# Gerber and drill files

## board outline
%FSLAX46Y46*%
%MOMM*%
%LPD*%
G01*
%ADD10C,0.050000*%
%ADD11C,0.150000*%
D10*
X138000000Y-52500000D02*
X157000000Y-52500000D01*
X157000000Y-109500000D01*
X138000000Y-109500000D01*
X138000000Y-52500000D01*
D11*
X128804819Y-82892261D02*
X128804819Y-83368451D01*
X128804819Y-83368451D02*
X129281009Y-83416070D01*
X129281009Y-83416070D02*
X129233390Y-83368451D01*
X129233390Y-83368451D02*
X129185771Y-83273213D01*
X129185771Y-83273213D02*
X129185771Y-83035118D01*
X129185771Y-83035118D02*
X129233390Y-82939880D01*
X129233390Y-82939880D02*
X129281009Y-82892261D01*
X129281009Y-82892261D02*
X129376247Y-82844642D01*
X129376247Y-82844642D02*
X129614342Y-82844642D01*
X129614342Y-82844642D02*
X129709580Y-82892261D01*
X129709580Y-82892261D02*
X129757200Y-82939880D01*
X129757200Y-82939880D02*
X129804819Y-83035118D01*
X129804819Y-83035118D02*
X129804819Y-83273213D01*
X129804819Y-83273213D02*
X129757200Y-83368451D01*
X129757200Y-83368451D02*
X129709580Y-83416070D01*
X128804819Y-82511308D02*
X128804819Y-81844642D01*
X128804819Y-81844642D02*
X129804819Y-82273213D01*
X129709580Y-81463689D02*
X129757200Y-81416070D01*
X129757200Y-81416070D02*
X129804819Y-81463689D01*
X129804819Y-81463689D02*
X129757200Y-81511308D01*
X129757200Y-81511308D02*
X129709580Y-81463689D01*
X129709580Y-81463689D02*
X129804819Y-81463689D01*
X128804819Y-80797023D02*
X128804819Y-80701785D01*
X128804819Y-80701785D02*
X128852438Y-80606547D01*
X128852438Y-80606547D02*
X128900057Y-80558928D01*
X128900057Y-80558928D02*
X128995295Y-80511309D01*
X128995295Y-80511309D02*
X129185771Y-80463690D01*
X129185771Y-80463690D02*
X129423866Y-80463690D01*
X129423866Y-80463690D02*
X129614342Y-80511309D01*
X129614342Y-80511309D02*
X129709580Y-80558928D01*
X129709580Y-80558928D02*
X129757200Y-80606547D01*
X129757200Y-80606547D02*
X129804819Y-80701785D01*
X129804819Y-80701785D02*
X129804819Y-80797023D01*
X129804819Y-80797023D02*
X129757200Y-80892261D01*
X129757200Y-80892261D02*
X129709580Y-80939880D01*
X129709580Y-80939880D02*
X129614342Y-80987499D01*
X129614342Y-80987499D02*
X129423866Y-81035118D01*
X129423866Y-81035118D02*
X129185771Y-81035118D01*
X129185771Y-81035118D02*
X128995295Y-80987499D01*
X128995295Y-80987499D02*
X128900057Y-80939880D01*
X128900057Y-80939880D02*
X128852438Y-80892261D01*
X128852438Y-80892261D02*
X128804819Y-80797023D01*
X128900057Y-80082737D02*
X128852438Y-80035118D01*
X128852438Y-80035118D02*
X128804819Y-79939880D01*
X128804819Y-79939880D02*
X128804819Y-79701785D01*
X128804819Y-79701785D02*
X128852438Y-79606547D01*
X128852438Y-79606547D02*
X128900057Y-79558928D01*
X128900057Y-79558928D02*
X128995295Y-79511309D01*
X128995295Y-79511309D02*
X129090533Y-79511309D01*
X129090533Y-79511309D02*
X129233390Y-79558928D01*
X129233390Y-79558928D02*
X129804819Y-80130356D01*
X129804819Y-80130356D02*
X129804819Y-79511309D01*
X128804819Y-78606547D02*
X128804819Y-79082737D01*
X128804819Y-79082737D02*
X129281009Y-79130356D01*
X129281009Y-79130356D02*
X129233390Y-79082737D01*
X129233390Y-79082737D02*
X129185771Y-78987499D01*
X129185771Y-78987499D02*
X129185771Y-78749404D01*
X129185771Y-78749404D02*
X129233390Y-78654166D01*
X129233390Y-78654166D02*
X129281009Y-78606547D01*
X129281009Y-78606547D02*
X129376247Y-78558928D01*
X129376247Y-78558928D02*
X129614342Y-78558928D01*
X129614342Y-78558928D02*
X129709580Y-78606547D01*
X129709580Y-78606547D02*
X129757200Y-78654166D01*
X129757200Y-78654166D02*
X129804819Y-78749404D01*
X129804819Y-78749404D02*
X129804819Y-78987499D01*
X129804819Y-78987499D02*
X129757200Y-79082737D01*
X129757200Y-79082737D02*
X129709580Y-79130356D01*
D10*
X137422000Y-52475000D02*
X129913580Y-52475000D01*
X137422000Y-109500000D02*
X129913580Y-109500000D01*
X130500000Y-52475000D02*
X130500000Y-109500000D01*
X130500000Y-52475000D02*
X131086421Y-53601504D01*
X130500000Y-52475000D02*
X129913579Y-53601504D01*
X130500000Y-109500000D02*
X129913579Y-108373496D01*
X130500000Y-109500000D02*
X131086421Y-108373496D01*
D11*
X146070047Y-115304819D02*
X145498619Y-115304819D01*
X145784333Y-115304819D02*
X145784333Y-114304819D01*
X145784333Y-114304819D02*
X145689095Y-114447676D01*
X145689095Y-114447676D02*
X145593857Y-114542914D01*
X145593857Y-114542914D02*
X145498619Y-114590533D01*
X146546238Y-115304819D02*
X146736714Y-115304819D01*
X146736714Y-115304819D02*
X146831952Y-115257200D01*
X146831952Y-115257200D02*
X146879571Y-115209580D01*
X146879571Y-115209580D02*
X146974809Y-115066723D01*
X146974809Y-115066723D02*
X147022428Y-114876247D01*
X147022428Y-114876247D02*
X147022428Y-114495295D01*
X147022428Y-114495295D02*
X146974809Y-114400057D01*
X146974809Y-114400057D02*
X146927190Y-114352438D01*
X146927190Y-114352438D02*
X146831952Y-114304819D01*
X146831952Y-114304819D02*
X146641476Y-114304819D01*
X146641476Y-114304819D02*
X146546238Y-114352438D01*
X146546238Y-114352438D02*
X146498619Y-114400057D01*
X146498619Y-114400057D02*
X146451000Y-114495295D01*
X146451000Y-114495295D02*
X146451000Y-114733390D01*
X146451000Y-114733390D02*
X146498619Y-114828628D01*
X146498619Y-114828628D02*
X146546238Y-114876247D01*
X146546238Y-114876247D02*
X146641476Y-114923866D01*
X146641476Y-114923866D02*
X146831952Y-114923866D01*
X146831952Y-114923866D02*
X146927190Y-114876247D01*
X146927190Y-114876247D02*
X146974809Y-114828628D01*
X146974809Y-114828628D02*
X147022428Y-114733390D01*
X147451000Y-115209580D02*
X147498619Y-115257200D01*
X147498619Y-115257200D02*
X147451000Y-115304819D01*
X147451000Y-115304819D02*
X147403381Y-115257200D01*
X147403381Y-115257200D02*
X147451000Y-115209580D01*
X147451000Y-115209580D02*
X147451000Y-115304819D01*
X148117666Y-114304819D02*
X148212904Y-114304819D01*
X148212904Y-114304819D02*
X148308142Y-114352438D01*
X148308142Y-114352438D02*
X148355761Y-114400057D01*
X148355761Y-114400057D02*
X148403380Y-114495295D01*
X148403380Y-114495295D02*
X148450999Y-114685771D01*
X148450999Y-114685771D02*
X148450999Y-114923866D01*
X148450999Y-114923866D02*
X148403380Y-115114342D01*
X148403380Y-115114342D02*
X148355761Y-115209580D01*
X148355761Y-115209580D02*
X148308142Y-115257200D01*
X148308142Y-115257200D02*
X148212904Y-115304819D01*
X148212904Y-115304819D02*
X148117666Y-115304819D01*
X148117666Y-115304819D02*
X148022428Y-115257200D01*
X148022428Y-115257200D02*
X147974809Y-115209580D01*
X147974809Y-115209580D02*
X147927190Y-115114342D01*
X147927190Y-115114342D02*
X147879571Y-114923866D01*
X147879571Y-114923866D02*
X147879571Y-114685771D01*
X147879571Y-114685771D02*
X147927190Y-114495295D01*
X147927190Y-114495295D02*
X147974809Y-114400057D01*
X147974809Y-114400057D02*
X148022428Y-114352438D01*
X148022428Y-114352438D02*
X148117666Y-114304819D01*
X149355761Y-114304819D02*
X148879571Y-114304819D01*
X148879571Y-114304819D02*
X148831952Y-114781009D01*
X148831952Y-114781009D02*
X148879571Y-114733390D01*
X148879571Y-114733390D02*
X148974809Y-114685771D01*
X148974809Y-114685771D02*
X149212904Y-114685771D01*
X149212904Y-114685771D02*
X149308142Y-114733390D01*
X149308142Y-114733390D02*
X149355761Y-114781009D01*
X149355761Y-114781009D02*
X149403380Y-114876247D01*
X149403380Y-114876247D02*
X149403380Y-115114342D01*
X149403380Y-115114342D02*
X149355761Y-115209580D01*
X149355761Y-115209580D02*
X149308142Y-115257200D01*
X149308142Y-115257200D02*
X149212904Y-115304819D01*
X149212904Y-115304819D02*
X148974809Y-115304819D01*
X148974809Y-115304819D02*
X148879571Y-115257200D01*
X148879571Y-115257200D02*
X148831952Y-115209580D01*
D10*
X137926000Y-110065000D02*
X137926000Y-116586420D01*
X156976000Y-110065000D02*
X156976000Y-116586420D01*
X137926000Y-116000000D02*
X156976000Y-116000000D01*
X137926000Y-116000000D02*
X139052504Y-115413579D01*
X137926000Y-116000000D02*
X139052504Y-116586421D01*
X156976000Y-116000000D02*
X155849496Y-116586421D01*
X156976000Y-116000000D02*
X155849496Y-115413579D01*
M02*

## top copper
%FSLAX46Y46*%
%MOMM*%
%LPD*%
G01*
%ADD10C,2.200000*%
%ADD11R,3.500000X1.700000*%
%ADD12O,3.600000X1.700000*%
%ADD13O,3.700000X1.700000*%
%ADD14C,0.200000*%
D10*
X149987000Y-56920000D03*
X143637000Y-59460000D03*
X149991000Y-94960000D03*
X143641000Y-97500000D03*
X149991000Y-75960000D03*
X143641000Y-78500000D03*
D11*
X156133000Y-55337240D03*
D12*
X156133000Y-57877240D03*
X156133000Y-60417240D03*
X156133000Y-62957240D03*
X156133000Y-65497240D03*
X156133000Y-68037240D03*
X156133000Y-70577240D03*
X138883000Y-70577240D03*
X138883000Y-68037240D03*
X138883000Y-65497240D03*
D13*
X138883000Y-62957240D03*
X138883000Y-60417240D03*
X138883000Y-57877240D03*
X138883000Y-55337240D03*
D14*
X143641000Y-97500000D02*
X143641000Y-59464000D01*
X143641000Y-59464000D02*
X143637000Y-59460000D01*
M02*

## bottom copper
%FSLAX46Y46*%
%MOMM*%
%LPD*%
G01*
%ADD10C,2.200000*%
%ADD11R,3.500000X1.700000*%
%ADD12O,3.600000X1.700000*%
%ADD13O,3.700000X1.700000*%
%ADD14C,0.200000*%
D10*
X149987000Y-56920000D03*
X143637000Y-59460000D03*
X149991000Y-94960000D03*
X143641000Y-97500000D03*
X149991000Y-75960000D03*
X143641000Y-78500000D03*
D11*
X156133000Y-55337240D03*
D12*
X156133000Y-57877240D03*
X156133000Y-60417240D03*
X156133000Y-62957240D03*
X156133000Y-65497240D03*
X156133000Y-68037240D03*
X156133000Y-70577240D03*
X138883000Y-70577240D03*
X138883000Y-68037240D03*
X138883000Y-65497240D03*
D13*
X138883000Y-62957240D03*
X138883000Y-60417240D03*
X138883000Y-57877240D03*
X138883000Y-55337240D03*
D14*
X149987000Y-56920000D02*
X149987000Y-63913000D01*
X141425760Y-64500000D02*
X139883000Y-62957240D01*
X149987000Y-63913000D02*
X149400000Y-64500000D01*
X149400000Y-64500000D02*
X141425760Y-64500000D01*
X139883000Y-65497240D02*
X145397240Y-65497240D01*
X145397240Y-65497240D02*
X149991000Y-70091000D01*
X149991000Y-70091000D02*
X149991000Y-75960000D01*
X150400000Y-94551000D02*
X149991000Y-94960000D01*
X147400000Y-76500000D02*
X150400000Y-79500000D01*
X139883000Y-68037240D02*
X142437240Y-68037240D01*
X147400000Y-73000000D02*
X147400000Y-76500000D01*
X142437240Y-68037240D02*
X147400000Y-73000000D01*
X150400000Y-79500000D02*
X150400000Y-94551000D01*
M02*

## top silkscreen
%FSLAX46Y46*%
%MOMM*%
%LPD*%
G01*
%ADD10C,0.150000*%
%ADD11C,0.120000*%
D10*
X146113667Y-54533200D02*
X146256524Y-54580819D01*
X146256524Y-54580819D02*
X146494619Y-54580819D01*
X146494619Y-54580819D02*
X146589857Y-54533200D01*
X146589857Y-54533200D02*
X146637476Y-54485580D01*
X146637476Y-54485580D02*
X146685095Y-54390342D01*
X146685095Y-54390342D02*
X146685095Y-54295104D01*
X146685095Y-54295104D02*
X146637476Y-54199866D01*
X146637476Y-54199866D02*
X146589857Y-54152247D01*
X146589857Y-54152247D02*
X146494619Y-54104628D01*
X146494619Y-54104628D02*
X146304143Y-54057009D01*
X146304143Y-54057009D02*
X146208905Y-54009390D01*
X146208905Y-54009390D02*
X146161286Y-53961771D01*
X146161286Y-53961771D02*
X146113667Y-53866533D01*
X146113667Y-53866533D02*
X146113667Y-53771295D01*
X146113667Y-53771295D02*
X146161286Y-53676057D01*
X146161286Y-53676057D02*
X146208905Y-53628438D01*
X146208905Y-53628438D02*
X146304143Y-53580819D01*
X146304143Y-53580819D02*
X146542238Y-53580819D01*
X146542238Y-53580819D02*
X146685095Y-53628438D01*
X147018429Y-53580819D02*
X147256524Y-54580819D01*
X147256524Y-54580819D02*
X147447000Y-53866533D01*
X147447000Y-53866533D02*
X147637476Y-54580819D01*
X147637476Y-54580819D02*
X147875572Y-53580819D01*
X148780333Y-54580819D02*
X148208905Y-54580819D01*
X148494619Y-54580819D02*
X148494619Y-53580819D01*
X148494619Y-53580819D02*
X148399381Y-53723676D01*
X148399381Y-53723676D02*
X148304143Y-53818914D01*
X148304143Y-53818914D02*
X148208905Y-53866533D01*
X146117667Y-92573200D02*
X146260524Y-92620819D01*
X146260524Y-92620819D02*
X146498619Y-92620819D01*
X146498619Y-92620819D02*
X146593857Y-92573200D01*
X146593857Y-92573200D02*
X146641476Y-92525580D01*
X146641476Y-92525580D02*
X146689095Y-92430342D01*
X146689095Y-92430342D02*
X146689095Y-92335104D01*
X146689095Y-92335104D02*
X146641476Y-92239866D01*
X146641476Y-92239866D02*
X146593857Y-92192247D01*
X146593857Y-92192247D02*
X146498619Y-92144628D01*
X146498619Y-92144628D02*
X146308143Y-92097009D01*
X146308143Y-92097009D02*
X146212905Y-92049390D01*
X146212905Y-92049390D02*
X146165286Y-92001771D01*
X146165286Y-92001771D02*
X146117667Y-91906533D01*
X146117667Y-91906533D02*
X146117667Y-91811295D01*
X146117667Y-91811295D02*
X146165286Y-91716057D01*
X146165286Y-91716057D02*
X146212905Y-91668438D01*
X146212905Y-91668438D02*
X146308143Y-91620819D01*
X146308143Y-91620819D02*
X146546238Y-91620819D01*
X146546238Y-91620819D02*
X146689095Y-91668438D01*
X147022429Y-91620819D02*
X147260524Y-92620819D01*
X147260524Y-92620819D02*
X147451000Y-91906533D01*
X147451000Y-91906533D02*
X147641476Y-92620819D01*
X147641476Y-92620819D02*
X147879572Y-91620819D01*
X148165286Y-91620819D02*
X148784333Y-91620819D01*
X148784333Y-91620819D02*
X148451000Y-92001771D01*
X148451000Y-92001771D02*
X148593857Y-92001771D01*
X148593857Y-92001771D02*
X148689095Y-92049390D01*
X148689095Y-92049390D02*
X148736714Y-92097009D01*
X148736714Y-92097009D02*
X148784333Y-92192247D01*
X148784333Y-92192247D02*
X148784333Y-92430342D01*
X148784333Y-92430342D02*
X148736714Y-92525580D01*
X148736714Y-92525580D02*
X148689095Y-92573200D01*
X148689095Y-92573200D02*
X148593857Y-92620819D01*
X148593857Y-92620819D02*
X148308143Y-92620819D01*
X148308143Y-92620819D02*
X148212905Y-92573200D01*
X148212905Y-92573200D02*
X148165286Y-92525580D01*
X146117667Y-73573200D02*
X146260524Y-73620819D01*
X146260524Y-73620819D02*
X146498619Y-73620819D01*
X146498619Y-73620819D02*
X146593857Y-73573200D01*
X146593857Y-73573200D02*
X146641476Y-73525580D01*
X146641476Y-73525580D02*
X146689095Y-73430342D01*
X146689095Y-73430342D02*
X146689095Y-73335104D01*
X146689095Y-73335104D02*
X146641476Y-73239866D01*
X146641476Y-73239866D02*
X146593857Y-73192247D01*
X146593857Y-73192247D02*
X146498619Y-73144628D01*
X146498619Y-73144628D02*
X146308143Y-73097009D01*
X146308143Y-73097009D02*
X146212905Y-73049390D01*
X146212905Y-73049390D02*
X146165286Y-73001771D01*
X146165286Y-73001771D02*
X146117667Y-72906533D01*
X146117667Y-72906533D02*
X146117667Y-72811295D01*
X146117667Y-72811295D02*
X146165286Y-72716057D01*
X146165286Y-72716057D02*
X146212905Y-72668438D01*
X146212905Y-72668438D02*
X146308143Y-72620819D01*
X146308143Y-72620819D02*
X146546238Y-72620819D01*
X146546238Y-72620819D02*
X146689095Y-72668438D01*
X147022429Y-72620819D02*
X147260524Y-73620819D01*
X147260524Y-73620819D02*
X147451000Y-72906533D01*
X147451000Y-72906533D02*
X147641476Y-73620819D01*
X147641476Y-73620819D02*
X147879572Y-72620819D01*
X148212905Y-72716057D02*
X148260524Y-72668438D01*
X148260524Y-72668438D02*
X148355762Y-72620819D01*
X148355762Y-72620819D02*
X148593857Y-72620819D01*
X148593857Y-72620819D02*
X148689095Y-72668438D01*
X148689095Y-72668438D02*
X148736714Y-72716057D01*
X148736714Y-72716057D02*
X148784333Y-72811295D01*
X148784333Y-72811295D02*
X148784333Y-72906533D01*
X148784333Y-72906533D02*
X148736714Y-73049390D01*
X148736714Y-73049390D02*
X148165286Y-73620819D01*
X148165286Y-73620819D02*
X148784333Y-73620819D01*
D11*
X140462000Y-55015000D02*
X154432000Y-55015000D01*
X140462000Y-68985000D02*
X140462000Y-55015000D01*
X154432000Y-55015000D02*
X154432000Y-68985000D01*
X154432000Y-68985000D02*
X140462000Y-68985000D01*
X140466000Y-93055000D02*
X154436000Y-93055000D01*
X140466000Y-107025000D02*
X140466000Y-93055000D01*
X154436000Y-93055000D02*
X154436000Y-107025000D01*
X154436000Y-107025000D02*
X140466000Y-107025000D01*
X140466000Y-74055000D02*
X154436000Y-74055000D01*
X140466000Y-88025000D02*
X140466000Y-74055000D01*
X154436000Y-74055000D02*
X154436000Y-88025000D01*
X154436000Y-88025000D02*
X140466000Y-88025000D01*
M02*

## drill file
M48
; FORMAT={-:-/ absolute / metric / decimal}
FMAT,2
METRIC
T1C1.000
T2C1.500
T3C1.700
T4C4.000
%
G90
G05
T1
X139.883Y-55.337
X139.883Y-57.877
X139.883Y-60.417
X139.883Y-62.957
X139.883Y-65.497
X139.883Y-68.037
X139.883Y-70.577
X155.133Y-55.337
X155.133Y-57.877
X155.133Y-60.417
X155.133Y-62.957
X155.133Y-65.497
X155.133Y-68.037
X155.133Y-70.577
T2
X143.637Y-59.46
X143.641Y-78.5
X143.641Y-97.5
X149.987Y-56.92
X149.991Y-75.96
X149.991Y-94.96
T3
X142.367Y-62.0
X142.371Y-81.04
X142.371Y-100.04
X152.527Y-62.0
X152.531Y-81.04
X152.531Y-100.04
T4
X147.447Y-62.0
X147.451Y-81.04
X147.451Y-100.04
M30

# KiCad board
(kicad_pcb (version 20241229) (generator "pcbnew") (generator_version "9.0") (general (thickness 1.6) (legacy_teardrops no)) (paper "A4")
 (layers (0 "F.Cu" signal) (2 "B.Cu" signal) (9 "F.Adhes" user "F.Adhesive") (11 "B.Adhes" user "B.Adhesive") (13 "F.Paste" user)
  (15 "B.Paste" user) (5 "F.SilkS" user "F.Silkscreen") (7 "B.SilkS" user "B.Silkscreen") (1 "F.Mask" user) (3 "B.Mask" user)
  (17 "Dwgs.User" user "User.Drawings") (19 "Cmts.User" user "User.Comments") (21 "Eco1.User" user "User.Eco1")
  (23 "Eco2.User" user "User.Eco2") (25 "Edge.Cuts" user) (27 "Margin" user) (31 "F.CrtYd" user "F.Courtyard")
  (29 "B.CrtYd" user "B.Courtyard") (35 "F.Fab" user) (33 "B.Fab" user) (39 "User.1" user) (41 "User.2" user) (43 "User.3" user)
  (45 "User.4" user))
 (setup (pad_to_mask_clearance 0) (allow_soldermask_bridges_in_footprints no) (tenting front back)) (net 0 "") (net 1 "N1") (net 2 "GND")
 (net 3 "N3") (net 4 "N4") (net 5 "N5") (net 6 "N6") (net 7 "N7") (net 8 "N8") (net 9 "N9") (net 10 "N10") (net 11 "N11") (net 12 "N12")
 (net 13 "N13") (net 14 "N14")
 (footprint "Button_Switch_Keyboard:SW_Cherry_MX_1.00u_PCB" (layer "F.Cu") (at 149.987 56.92)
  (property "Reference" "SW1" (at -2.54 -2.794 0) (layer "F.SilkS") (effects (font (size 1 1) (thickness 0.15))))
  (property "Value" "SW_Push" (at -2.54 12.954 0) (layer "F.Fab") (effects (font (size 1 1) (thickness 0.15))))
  (fp_line (start -9.525 -1.905) (end 4.445 -1.905) (stroke (width 0.12) (type solid)) (layer "F.SilkS"))
  (fp_line (start -9.525 12.065) (end -9.525 -1.905) (stroke (width 0.12) (type solid)) (layer "F.SilkS"))
  (fp_line (start 4.445 -1.905) (end 4.445 12.065) (stroke (width 0.12) (type solid)) (layer "F.SilkS"))
  (fp_line (start 4.445 12.065) (end -9.525 12.065) (stroke (width 0.12) (type solid)) (layer "F.SilkS"))
  (pad "" np_thru_hole circle (at -7.62 5.08) (size 1.7 1.7) (drill 1.7) (layers "*.Cu" "*.Mask"))
  (pad "" np_thru_hole circle (at -2.54 5.08) (size 4 4) (drill 4) (layers "*.Cu" "*.Mask"))
  (pad "" np_thru_hole circle (at 2.54 5.08) (size 1.7 1.7) (drill 1.7) (layers "*.Cu" "*.Mask"))
  (pad "1" thru_hole circle (at 0 0) (size 2.2 2.2) (drill 1.5) (layers "*.Cu" "*.Mask") (remove_unused_layers no) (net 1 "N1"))
  (pad "2" thru_hole circle (at -6.35 2.54) (size 2.2 2.2) (drill 1.5) (layers "*.Cu" "*.Mask") (remove_unused_layers no) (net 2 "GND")))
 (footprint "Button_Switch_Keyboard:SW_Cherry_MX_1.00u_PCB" (layer "F.Cu") (at 149.991 94.96)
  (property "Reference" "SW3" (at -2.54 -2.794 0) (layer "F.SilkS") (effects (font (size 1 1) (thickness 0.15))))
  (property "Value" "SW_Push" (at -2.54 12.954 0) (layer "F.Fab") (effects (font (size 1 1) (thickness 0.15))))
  (fp_line (start -9.525 -1.905) (end 4.445 -1.905) (stroke (width 0.12) (type solid)) (layer "F.SilkS"))
  (fp_line (start -9.525 12.065) (end -9.525 -1.905) (stroke (width 0.12) (type solid)) (layer "F.SilkS"))
  (fp_line (start 4.445 -1.905) (end 4.445 12.065) (stroke (width 0.12) (type solid)) (layer "F.SilkS"))
  (fp_line (start 4.445 12.065) (end -9.525 12.065) (stroke (width 0.12) (type solid)) (layer "F.SilkS"))
  (pad "" np_thru_hole circle (at -7.62 5.08) (size 1.7 1.7) (drill 1.7) (layers "*.Cu" "*.Mask"))
  (pad "" np_thru_hole circle (at -2.54 5.08) (size 4 4) (drill 4) (layers "*.Cu" "*.Mask"))
  (pad "" np_thru_hole circle (at 2.54 5.08) (size 1.7 1.7) (drill 1.7) (layers "*.Cu" "*.Mask"))
  (pad "1" thru_hole circle (at 0 0) (size 2.2 2.2) (drill 1.5) (layers "*.Cu" "*.Mask") (remove_unused_layers no) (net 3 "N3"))
  (pad "2" thru_hole circle (at -6.35 2.54) (size 2.2 2.2) (drill 1.5) (layers "*.Cu" "*.Mask") (remove_unused_layers no) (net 2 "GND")))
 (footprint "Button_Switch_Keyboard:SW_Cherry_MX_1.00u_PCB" (layer "F.Cu") (at 149.991 75.96)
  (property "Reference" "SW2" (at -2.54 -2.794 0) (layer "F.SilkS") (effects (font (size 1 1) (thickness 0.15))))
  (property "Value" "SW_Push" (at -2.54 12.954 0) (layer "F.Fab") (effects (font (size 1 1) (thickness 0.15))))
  (fp_line (start -9.525 -1.905) (end 4.445 -1.905) (stroke (width 0.12) (type solid)) (layer "F.SilkS"))
  (fp_line (start -9.525 12.065) (end -9.525 -1.905) (stroke (width 0.12) (type solid)) (layer "F.SilkS"))
  (fp_line (start 4.445 -1.905) (end 4.445 12.065) (stroke (width 0.12) (type solid)) (layer "F.SilkS"))
  (fp_line (start 4.445 12.065) (end -9.525 12.065) (stroke (width 0.12) (type solid)) (layer "F.SilkS"))
  (pad "" np_thru_hole circle (at -7.62 5.08) (size 1.7 1.7) (drill 1.7) (layers "*.Cu" "*.Mask"))
  (pad "" np_thru_hole circle (at -2.54 5.08) (size 4 4) (drill 4) (layers "*.Cu" "*.Mask"))
  (pad "" np_thru_hole circle (at 2.54 5.08) (size 1.7 1.7) (drill 1.7) (layers "*.Cu" "*.Mask"))
  (pad "1" thru_hole circle (at 0 0) (size 2.2 2.2) (drill 1.5) (layers "*.Cu" "*.Mask") (remove_unused_layers no) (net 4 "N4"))
  (pad "2" thru_hole circle (at -6.35 2.54) (size 2.2 2.2) (drill 1.5) (layers "*.Cu" "*.Mask") (remove_unused_layers no) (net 2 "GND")))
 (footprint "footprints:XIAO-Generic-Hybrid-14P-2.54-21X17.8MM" (layer "B.Cu") (at 147.508 62.95724 180)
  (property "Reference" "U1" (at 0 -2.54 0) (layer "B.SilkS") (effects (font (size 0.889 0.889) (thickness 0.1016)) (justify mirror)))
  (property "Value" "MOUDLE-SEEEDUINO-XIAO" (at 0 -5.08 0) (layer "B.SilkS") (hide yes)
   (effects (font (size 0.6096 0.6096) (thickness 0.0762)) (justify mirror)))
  (pad "1" thru_hole rect (at -7.625 7.62 180) (size 3.5 1.7) (drill 1 (offset -1 0)) (layers "*.Cu" "*.Mask") (remove_unused_layers no)
   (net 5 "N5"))
  (pad "2" thru_hole oval (at -7.625 5.08 180) (size 3.6 1.7) (drill 1 (offset -1 0)) (layers "*.Cu" "*.Mask") (remove_unused_layers no)
   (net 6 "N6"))
  (pad "3" thru_hole oval (at -7.625 2.54 180) (size 3.6 1.7) (drill 1 (offset -1 0)) (layers "*.Cu" "*.Mask") (remove_unused_layers no)
   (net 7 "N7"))
  (pad "4" thru_hole oval (at -7.625 0 180) (size 3.6 1.7) (drill 1 (offset -1 0)) (layers "*.Cu" "*.Mask") (remove_unused_layers no)
   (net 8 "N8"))
  (pad "5" thru_hole oval (at -7.625 -2.54 180) (size 3.6 1.7) (drill 1 (offset -1 0)) (layers "*.Cu" "*.Mask") (remove_unused_layers no)
   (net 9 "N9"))
  (pad "6" thru_hole oval (at -7.625 -5.08) (size 3.6 1.7) (drill 1 (offset 1 0)) (layers "*.Cu" "*.Mask") (remove_unused_layers no)
   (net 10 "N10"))
  (pad "7" thru_hole oval (at -7.625 -7.62 180) (size 3.6 1.7) (drill 1 (offset -1 0)) (layers "*.Cu" "*.Mask") (remove_unused_layers no)
   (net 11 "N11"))
  (pad "8" thru_hole oval (at 7.625 -7.62 180) (size 3.6 1.7) (drill 1 (offset 1 0)) (layers "*.Cu" "*.Mask") (remove_unused_layers no)
   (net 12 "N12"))
  (pad "9" thru_hole oval (at 7.625 -5.08 180) (size 3.6 1.7) (drill 1 (offset 1 0)) (layers "*.Cu" "*.Mask") (remove_unused_layers no)
   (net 3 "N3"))
  (pad "10" thru_hole oval (at 7.625 -2.54 180) (size 3.6 1.7) (drill 1 (offset 1 0)) (layers "*.Cu" "*.Mask") (remove_unused_layers no)
   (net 4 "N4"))
  (pad "11" thru_hole oval (at 7.625 0 180) (size 3.7 1.7) (drill 1 (offset 1 0)) (layers "*.Cu" "*.Mask") (remove_unused_layers no)
   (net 1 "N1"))
  (pad "12" thru_hole oval (at 7.625 2.54 180) (size 3.7 1.7) (drill 1 (offset 1 0)) (layers "*.Cu" "*.Mask") (remove_unused_layers no)
   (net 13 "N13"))
  (pad "13" thru_hole oval (at 7.625 5.08 180) (size 3.7 1.7) (drill 1 (offset 1 0)) (layers "*.Cu" "*.Mask") (remove_unused_layers no)
   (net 2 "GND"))
  (pad "14" thru_hole oval (at 7.625 7.62 180) (size 3.7 1.7) (drill 1 (offset 1 0)) (layers "*.Cu" "*.Mask") (remove_unused_layers no)
   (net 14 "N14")))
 (gr_rect (start 138 52.5) (end 157 109.5) (stroke (width 0.05) (type default)) (fill no) (layer "Edge.Cuts"))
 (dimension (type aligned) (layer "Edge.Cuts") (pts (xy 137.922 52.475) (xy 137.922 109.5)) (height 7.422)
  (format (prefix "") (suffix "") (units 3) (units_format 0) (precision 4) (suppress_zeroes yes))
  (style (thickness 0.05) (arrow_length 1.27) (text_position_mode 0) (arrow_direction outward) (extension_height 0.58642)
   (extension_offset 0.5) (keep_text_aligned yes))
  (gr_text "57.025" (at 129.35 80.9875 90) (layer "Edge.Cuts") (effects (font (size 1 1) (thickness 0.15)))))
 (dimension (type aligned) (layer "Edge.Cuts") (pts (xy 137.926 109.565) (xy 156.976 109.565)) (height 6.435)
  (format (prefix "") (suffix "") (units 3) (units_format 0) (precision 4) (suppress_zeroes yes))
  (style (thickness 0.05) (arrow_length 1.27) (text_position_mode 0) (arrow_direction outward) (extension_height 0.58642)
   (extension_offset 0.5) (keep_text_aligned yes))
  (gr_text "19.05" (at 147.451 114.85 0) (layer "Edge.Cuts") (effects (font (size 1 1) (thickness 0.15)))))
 (segment (start 143.641 97.5) (end 143.641 59.464) (width 0.2) (layer "F.Cu") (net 2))
 (segment (start 143.641 59.464) (end 143.637 59.46) (width 0.2) (layer "F.Cu") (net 2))
 (segment (start 149.987 56.92) (end 149.987 63.913) (width 0.2) (layer "B.Cu") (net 1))
 (segment (start 141.42576 64.5) (end 139.883 62.95724) (width 0.2) (layer "B.Cu") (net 1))
 (segment (start 149.987 63.913) (end 149.4 64.5) (width 0.2) (layer "B.Cu") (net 1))
 (segment (start 149.4 64.5) (end 141.42576 64.5) (width 0.2) (layer "B.Cu") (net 1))
 (segment (start 139.883 65.49724) (end 145.39724 65.49724) (width 0.2) (layer "B.Cu") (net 4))
 (segment (start 145.39724 65.49724) (end 149.991 70.091) (width 0.2) (layer "B.Cu") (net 4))
 (segment (start 149.991 70.091) (end 149.991 75.96) (width 0.2) (layer "B.Cu") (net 4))
 (segment (start 150.4 94.551) (end 149.991 94.96) (width 0.2) (layer "B.Cu") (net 3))
 (segment (start 147.4 76.5) (end 150.4 79.5) (width 0.2) (layer "B.Cu") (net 3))
 (segment (start 139.883 68.03724) (end 142.43724 68.03724) (width 0.2) (layer "B.Cu") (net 3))
 (segment (start 147.4 73) (end 147.4 76.5) (width 0.2) (layer "B.Cu") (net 3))
 (segment (start 142.43724 68.03724) (end 147.4 73) (width 0.2) (layer "B.Cu") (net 3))
 (segment (start 150.4 79.5) (end 150.4 94.551) (width 0.2) (layer "B.Cu") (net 3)))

